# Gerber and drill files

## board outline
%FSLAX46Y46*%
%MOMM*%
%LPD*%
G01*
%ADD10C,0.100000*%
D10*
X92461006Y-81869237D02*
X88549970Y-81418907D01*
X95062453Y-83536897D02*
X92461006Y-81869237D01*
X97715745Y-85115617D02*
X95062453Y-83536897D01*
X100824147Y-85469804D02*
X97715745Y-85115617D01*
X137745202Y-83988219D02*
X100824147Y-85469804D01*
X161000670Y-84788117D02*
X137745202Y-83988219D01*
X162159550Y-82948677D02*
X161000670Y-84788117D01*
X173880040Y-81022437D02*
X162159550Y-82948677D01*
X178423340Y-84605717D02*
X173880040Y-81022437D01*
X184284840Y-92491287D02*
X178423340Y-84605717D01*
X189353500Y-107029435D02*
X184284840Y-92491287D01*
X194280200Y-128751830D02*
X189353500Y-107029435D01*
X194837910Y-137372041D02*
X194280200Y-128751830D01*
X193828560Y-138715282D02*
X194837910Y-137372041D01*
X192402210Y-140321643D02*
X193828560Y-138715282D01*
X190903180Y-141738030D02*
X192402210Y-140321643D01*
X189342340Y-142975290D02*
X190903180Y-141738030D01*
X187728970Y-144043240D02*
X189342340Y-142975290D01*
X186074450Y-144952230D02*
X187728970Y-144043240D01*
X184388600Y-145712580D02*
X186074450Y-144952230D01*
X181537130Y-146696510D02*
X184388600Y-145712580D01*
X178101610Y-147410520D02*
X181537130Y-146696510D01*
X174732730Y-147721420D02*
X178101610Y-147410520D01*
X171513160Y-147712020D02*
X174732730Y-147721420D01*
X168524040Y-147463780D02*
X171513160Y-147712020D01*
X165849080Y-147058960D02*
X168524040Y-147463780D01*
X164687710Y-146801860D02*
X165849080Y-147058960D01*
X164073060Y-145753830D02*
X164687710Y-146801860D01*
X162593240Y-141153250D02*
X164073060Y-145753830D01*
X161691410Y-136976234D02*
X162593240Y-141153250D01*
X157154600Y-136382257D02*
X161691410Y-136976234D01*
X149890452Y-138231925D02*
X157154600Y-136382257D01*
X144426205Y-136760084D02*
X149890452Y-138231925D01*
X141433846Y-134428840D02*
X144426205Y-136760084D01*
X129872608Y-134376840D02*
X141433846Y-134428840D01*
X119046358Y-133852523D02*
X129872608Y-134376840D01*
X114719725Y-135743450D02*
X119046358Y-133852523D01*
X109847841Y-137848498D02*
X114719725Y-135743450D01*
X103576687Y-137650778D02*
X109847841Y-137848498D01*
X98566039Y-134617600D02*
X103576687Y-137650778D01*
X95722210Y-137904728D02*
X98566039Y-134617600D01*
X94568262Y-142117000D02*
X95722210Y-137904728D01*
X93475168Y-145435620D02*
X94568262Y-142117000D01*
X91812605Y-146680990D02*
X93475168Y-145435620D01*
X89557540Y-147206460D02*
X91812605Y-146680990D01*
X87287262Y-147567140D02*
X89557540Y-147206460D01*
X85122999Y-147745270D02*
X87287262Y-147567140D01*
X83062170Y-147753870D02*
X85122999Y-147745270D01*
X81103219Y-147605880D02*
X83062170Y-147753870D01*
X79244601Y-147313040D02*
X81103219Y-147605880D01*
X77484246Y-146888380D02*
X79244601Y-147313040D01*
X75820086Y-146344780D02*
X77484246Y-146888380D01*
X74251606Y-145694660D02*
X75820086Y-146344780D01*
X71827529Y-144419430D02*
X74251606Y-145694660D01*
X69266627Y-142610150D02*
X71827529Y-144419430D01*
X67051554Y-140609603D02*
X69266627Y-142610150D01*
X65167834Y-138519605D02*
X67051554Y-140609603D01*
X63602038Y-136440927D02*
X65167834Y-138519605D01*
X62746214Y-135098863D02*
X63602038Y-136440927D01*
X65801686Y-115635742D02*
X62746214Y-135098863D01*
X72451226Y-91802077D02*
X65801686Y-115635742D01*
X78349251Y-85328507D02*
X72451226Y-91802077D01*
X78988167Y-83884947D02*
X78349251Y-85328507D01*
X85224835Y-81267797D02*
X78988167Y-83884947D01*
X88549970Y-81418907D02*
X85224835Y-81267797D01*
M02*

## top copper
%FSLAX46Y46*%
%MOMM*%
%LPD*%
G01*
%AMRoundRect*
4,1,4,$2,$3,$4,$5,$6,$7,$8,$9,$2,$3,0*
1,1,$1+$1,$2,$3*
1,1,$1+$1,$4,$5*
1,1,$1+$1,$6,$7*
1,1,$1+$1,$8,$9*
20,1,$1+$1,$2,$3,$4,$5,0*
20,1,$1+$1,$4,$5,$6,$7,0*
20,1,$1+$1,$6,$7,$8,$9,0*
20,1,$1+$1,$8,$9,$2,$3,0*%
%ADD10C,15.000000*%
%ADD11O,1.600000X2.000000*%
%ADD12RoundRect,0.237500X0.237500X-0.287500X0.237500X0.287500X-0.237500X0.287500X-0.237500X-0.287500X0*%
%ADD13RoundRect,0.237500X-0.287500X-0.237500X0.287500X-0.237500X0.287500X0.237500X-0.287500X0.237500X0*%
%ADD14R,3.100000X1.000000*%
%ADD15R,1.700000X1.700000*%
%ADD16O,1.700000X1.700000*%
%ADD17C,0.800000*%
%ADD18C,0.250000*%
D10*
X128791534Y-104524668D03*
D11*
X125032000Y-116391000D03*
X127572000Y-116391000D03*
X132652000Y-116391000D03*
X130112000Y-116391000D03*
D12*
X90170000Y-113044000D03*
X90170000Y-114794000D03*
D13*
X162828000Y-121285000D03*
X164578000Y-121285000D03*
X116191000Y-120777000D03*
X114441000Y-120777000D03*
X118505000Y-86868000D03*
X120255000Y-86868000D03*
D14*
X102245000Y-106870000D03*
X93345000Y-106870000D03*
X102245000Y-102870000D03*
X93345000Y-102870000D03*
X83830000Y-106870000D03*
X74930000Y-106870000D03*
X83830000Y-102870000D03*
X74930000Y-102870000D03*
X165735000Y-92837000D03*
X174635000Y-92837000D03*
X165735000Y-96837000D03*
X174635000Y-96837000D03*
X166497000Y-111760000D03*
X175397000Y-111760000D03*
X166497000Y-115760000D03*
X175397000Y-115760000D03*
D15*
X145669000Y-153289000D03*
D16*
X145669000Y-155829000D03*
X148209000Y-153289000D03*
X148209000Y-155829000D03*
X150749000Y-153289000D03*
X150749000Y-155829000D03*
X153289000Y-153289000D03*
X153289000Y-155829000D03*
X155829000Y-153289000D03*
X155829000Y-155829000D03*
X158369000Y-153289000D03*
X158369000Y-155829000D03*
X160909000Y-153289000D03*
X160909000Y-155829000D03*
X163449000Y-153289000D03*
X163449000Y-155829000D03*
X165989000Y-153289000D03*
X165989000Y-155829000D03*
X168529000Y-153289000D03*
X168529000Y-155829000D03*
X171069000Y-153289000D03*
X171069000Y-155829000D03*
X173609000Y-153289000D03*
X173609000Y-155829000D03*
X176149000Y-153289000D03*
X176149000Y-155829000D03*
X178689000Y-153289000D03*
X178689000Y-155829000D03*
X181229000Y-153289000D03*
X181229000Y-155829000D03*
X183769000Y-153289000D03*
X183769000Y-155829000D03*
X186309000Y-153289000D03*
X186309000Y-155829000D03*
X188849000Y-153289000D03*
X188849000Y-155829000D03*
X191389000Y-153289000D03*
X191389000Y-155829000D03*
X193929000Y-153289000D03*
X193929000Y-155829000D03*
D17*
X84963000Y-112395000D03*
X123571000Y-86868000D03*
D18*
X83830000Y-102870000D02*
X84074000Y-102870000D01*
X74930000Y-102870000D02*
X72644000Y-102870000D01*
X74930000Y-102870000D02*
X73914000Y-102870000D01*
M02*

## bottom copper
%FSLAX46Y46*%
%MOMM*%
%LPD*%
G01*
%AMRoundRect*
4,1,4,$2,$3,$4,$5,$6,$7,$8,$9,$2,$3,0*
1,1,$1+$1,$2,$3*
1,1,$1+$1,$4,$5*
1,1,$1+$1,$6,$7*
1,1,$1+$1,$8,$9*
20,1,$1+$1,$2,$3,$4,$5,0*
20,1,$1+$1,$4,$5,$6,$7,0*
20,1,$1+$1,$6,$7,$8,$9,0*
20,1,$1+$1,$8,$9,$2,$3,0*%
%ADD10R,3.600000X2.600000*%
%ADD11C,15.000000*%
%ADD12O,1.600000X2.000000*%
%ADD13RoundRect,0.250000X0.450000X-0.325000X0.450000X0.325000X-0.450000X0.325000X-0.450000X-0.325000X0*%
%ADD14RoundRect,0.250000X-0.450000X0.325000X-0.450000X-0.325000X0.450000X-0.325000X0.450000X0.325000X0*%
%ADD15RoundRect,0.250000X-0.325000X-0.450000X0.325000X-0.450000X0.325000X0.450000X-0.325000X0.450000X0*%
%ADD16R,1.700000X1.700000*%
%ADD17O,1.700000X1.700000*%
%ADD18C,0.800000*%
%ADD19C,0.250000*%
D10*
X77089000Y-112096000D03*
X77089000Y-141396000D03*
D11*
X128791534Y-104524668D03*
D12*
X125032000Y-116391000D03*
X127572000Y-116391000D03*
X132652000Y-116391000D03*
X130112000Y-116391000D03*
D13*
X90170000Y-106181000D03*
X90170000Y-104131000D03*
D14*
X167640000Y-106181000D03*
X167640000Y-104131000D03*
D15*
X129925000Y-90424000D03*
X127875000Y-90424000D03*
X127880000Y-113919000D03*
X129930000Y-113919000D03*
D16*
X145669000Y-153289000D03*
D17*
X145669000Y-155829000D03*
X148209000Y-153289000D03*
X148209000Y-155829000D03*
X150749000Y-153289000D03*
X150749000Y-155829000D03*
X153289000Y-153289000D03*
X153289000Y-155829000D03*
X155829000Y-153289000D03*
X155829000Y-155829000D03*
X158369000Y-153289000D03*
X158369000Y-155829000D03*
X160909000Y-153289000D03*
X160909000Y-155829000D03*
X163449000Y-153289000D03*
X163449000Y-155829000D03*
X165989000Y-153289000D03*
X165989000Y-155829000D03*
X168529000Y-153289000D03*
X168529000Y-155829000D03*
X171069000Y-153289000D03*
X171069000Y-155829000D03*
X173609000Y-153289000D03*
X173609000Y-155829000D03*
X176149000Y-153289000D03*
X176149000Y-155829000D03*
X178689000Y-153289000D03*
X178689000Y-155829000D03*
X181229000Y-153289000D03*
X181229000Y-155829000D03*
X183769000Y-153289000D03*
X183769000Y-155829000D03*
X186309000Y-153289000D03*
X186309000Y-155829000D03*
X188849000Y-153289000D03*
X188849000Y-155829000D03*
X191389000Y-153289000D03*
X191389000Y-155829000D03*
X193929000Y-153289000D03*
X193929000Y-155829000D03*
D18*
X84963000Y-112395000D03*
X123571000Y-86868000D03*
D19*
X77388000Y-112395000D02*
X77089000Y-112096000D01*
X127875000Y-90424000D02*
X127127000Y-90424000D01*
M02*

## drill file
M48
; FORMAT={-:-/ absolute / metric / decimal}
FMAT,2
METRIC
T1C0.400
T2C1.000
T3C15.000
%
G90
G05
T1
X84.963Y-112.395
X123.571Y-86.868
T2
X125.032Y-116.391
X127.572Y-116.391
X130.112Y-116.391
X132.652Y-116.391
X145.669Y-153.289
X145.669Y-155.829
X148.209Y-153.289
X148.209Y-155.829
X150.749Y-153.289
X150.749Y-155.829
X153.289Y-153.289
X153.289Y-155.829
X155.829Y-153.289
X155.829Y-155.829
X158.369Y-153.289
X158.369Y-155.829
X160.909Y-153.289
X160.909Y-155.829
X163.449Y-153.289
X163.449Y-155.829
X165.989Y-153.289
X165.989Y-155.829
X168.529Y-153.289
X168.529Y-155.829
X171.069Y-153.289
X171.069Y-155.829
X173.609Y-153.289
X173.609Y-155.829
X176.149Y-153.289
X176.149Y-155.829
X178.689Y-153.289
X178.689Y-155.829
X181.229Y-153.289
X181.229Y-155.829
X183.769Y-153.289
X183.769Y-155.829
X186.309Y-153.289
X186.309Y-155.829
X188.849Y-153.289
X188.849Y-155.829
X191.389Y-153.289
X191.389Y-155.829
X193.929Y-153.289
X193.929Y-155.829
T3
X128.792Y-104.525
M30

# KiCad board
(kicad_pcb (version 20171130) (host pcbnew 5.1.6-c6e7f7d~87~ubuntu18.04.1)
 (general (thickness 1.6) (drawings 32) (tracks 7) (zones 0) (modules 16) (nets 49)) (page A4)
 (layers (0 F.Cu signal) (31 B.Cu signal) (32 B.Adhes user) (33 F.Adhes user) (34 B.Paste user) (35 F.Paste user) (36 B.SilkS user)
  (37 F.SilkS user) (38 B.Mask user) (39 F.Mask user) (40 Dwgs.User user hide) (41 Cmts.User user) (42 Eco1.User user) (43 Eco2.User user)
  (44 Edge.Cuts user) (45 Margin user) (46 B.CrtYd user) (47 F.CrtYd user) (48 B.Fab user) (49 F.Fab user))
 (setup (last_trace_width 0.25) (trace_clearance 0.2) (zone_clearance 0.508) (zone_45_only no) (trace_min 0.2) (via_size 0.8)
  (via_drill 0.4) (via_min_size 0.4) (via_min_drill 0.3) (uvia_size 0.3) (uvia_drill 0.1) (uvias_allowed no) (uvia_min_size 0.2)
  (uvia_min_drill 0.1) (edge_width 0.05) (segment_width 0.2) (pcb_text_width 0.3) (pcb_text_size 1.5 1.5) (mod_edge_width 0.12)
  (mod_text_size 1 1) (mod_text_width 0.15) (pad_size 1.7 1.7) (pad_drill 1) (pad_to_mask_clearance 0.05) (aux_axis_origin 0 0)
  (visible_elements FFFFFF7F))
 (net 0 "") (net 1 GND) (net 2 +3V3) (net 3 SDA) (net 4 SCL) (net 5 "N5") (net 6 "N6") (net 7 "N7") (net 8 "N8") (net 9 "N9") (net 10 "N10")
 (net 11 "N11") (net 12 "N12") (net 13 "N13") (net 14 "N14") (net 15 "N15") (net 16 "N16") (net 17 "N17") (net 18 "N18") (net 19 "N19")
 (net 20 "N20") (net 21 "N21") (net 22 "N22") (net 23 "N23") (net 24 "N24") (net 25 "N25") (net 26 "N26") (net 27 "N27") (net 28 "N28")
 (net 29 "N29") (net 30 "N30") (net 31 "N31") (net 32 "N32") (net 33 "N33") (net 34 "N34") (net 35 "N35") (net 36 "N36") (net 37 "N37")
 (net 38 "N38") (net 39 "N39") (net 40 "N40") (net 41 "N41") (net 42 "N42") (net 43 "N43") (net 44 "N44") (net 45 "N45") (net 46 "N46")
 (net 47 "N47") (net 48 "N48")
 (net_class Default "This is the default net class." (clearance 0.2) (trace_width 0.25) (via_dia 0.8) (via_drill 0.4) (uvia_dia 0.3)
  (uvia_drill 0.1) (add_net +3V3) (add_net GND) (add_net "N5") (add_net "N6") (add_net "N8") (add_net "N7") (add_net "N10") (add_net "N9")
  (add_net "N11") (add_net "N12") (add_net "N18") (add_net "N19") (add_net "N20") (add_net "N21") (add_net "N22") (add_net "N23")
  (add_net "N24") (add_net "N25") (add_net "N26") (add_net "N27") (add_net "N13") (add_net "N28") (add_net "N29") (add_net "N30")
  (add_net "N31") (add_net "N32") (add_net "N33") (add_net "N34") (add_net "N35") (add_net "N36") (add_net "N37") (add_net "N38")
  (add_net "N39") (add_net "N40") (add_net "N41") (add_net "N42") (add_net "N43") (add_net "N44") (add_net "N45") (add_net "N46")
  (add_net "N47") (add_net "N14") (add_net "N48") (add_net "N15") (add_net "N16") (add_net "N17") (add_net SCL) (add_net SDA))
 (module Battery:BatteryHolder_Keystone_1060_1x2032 (layer B.Cu) (at 77.089 126.746 90)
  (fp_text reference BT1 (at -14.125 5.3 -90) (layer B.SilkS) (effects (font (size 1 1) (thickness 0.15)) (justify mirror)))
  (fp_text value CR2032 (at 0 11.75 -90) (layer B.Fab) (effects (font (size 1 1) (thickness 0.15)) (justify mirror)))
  (pad 2 smd rect (at 14.65 0 270) (size 2.6 3.6) (layers B.Cu B.Paste B.Mask) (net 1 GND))
  (pad 1 smd rect (at -14.65 0 270) (size 2.6 3.6) (layers B.Cu B.Paste B.Mask) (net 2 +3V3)))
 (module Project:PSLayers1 (layer F.Cu) (at 127 115.824)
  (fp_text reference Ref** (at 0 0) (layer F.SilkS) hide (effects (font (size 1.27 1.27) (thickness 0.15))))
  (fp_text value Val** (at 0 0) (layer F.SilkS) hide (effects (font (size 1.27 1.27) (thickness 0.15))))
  (fp_line (start -34.538994 -33.954763) (end -38.45003 -34.405093) (layer Edge.Cuts) (width 0.1))
  (fp_line (start -31.937547 -32.287103) (end -34.538994 -33.954763) (layer Edge.Cuts) (width 0.1))
  (fp_line (start -29.284255 -30.708383) (end -31.937547 -32.287103) (layer Edge.Cuts) (width 0.1))
  (fp_line (start -26.175853 -30.354196) (end -29.284255 -30.708383) (layer Edge.Cuts) (width 0.1))
  (fp_line (start 10.745202 -31.835781) (end -26.175853 -30.354196) (layer Edge.Cuts) (width 0.1))
  (fp_line (start 34.00067 -31.035883) (end 10.745202 -31.835781) (layer Edge.Cuts) (width 0.1))
  (fp_line (start 35.15955 -32.875323) (end 34.00067 -31.035883) (layer Edge.Cuts) (width 0.1))
  (fp_line (start 46.88004 -34.801563) (end 35.15955 -32.875323) (layer Edge.Cuts) (width 0.1))
  (fp_line (start 51.42334 -31.218283) (end 46.88004 -34.801563) (layer Edge.Cuts) (width 0.1))
  (fp_line (start 57.28484 -23.332713) (end 51.42334 -31.218283) (layer Edge.Cuts) (width 0.1))
  (fp_line (start 62.3535 -8.794565) (end 57.28484 -23.332713) (layer Edge.Cuts) (width 0.1))
  (fp_line (start 67.2802 12.92783) (end 62.3535 -8.794565) (layer Edge.Cuts) (width 0.1))
  (fp_line (start 67.83791 21.548041) (end 67.2802 12.92783) (layer Edge.Cuts) (width 0.1))
  (fp_line (start 66.82856 22.891282) (end 67.83791 21.548041) (layer Edge.Cuts) (width 0.1))
  (fp_line (start 65.40221 24.497643) (end 66.82856 22.891282) (layer Edge.Cuts) (width 0.1))
  (fp_line (start 63.90318 25.91403) (end 65.40221 24.497643) (layer Edge.Cuts) (width 0.1))
  (fp_line (start 62.34234 27.15129) (end 63.90318 25.91403) (layer Edge.Cuts) (width 0.1))
  (fp_line (start 60.72897 28.21924) (end 62.34234 27.15129) (layer Edge.Cuts) (width 0.1))
  (fp_line (start 59.07445 29.12823) (end 60.72897 28.21924) (layer Edge.Cuts) (width 0.1))
  (fp_line (start 57.3886 29.88858) (end 59.07445 29.12823) (layer Edge.Cuts) (width 0.1))
  (fp_line (start 54.53713 30.87251) (end 57.3886 29.88858) (layer Edge.Cuts) (width 0.1))
  (fp_line (start 51.10161 31.58652) (end 54.53713 30.87251) (layer Edge.Cuts) (width 0.1))
  (fp_line (start 47.73273 31.89742) (end 51.10161 31.58652) (layer Edge.Cuts) (width 0.1))
  (fp_line (start 44.51316 31.88802) (end 47.73273 31.89742) (layer Edge.Cuts) (width 0.1))
  (fp_line (start 41.52404 31.63978) (end 44.51316 31.88802) (layer Edge.Cuts) (width 0.1))
  (fp_line (start 38.84908 31.23496) (end 41.52404 31.63978) (layer Edge.Cuts) (width 0.1))
  (fp_line (start 37.68771 30.97786) (end 38.84908 31.23496) (layer Edge.Cuts) (width 0.1))
  (fp_line (start 37.07306 29.92983) (end 37.68771 30.97786) (layer Edge.Cuts) (width 0.1))
  (fp_line (start 35.59324 25.32925) (end 37.07306 29.92983) (layer Edge.Cuts) (width 0.1))
  (fp_line (start 34.69141 21.152234) (end 35.59324 25.32925) (layer Edge.Cuts) (width 0.1))
  (fp_line (start 30.1546 20.558257) (end 34.69141 21.152234) (layer Edge.Cuts) (width 0.1))
  (fp_line (start 22.890452 22.407925) (end 30.1546 20.558257) (layer Edge.Cuts) (width 0.1))
  (fp_line (start 17.426205 20.936084) (end 22.890452 22.407925) (layer Edge.Cuts) (width 0.1))
  (fp_line (start 14.433846 18.60484) (end 17.426205 20.936084) (layer Edge.Cuts) (width 0.1))
  (fp_line (start 2.872608 18.55284) (end 14.433846 18.60484) (layer Edge.Cuts) (width 0.1))
  (fp_line (start -7.953642 18.028523) (end 2.872608 18.55284) (layer Edge.Cuts) (width 0.1))
  (fp_line (start -12.280275 19.91945) (end -7.953642 18.028523) (layer Edge.Cuts) (width 0.1))
  (fp_line (start -17.152159 22.024498) (end -12.280275 19.91945) (layer Edge.Cuts) (width 0.1))
  (fp_line (start -23.423313 21.826778) (end -17.152159 22.024498) (layer Edge.Cuts) (width 0.1))
  (fp_line (start -28.433961 18.7936) (end -23.423313 21.826778) (layer Edge.Cuts) (width 0.1))
  (fp_line (start -31.27779 22.080728) (end -28.433961 18.7936) (layer Edge.Cuts) (width 0.1))
  (fp_line (start -32.431738 26.293) (end -31.27779 22.080728) (layer Edge.Cuts) (width 0.1))
  (fp_line (start -33.524832 29.61162) (end -32.431738 26.293) (layer Edge.Cuts) (width 0.1))
  (fp_line (start -35.187395 30.85699) (end -33.524832 29.61162) (layer Edge.Cuts) (width 0.1))
  (fp_line (start -37.44246 31.38246) (end -35.187395 30.85699) (layer Edge.Cuts) (width 0.1))
  (fp_line (start -39.712738 31.74314) (end -37.44246 31.38246) (layer Edge.Cuts) (width 0.1))
  (fp_line (start -41.877001 31.92127) (end -39.712738 31.74314) (layer Edge.Cuts) (width 0.1))
  (fp_line (start -43.93783 31.92987) (end -41.877001 31.92127) (layer Edge.Cuts) (width 0.1))
  (fp_line (start -45.896781 31.78188) (end -43.93783 31.92987) (layer Edge.Cuts) (width 0.1))
  (fp_line (start -47.755399 31.48904) (end -45.896781 31.78188) (layer Edge.Cuts) (width 0.1))
  (fp_line (start -49.515754 31.06438) (end -47.755399 31.48904) (layer Edge.Cuts) (width 0.1))
  (fp_line (start -51.179914 30.52078) (end -49.515754 31.06438) (layer Edge.Cuts) (width 0.1))
  (fp_line (start -52.748394 29.87066) (end -51.179914 30.52078) (layer Edge.Cuts) (width 0.1))
  (fp_line (start -55.172471 28.59543) (end -52.748394 29.87066) (layer Edge.Cuts) (width 0.1))
  (fp_line (start -57.733373 26.78615) (end -55.172471 28.59543) (layer Edge.Cuts) (width 0.1))
  (fp_line (start -59.948446 24.785603) (end -57.733373 26.78615) (layer Edge.Cuts) (width 0.1))
  (fp_line (start -61.832166 22.695605) (end -59.948446 24.785603) (layer Edge.Cuts) (width 0.1))
  (fp_line (start -63.397962 20.616927) (end -61.832166 22.695605) (layer Edge.Cuts) (width 0.1))
  (fp_line (start -64.253786 19.274863) (end -63.397962 20.616927) (layer Edge.Cuts) (width 0.1))
  (fp_line (start -61.198314 -0.188258) (end -64.253786 19.274863) (layer Edge.Cuts) (width 0.1))
  (fp_line (start -54.548774 -24.021923) (end -61.198314 -0.188258) (layer Edge.Cuts) (width 0.1))
  (fp_line (start -48.650749 -30.495493) (end -54.548774 -24.021923) (layer Edge.Cuts) (width 0.1))
  (fp_line (start -48.011833 -31.939053) (end -48.650749 -30.495493) (layer Edge.Cuts) (width 0.1))
  (fp_line (start -41.775165 -34.556203) (end -48.011833 -31.939053) (layer Edge.Cuts) (width 0.1))
  (fp_line (start -38.45003 -34.405093) (end -41.775165 -34.556203) (layer Edge.Cuts) (width 0.1))
  (pad 1 thru_hole circle (at 1.791534 -11.299332) (size 15 15) (drill 15) (layers *.Cu *.Mask)))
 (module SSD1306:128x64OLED (layer F.Cu) (at 129.032 105.791 180)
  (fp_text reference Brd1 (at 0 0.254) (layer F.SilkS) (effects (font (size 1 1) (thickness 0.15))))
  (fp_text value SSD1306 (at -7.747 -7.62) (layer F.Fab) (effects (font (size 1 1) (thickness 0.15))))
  (pad 4 thru_hole oval (at 4 -10.6 270) (size 2 1.6) (drill 1) (layers *.Cu *.Mask) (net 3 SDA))
  (pad 3 thru_hole oval (at 1.46 -10.6 270) (size 2 1.6) (drill 1) (layers *.Cu *.Mask) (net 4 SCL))
  (pad 1 thru_hole oval (at -3.62 -10.6 270) (size 2 1.6) (drill 1) (layers *.Cu *.Mask) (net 1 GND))
  (pad 2 thru_hole oval (at -1.08 -10.6 270) (size 2 1.6) (drill 1) (layers *.Cu *.Mask) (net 2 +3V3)))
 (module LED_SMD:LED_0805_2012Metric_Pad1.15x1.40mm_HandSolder (layer B.Cu) (at 90.17 105.156 90)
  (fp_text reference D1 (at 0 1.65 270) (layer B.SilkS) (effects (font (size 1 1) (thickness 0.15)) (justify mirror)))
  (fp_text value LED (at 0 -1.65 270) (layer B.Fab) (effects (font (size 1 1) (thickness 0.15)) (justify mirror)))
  (pad 1 smd roundrect (at -1.025 0 90) (size 1.15 1.4) (layers B.Cu B.Paste B.Mask) (roundrect_rratio 0.217391) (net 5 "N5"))
  (pad 2 smd roundrect (at 1.025 0 90) (size 1.15 1.4) (layers B.Cu B.Paste B.Mask) (roundrect_rratio 0.217391) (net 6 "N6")))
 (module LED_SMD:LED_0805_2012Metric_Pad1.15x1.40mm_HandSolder (layer B.Cu) (at 167.64 105.156 270)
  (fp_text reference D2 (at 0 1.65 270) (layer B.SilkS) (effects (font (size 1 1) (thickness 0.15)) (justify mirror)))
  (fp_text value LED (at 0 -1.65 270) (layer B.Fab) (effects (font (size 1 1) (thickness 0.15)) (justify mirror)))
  (pad 2 smd roundrect (at 1.025 0 270) (size 1.15 1.4) (layers B.Cu B.Paste B.Mask) (roundrect_rratio 0.217391) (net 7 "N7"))
  (pad 1 smd roundrect (at -1.025 0 270) (size 1.15 1.4) (layers B.Cu B.Paste B.Mask) (roundrect_rratio 0.217391) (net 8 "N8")))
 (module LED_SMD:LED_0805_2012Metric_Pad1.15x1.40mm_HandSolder (layer B.Cu) (at 128.9 90.424)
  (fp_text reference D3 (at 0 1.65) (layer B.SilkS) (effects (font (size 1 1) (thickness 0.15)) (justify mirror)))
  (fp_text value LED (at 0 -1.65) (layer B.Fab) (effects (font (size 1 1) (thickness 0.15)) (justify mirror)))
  (pad 2 smd roundrect (at 1.025 0) (size 1.15 1.4) (layers B.Cu B.Paste B.Mask) (roundrect_rratio 0.217391) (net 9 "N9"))
  (pad 1 smd roundrect (at -1.025 0) (size 1.15 1.4) (layers B.Cu B.Paste B.Mask) (roundrect_rratio 0.217391) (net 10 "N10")))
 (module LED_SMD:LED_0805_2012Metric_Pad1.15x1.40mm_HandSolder (layer B.Cu) (at 128.905 113.919)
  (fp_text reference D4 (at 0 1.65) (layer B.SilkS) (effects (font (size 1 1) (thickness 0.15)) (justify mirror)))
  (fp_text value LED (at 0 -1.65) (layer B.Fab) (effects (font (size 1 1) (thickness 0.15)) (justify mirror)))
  (pad 1 smd roundrect (at -1.025 0) (size 1.15 1.4) (layers B.Cu B.Paste B.Mask) (roundrect_rratio 0.217391) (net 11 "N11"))
  (pad 2 smd roundrect (at 1.025 0) (size 1.15 1.4) (layers B.Cu B.Paste B.Mask) (roundrect_rratio 0.217391) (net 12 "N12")))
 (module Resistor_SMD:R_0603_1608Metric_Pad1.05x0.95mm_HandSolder (layer F.Cu) (at 90.17 113.919 90)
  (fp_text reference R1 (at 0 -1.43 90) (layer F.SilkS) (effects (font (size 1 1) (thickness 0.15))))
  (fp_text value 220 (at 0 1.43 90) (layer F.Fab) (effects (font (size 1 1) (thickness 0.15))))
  (pad 2 smd roundrect (at 0.875 0 90) (size 1.05 0.95) (layers F.Cu F.Paste F.Mask) (roundrect_rratio 0.25) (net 5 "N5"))
  (pad 1 smd roundrect (at -0.875 0 90) (size 1.05 0.95) (layers F.Cu F.Paste F.Mask) (roundrect_rratio 0.25) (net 1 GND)))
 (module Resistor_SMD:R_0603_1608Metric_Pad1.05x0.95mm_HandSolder (layer F.Cu) (at 163.703 121.285)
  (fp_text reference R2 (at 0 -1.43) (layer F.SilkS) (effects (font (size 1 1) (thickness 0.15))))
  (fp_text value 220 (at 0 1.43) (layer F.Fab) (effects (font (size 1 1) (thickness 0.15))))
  (pad 1 smd roundrect (at -0.875 0) (size 1.05 0.95) (layers F.Cu F.Paste F.Mask) (roundrect_rratio 0.25) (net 1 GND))
  (pad 2 smd roundrect (at 0.875 0) (size 1.05 0.95) (layers F.Cu F.Paste F.Mask) (roundrect_rratio 0.25) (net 8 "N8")))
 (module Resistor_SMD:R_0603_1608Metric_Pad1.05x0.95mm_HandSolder (layer F.Cu) (at 115.316 120.777)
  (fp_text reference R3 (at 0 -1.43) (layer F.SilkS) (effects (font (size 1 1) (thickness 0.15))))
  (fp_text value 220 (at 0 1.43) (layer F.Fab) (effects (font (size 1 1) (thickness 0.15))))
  (pad 2 smd roundrect (at 0.875 0) (size 1.05 0.95) (layers F.Cu F.Paste F.Mask) (roundrect_rratio 0.25) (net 11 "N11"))
  (pad 1 smd roundrect (at -0.875 0) (size 1.05 0.95) (layers F.Cu F.Paste F.Mask) (roundrect_rratio 0.25) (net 1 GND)))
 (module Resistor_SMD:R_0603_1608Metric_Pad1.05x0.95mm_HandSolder (layer F.Cu) (at 119.38 86.868)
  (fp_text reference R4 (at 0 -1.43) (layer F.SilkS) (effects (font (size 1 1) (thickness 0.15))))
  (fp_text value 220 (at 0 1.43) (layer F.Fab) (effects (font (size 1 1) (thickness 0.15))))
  (pad 1 smd roundrect (at -0.875 0) (size 1.05 0.95) (layers F.Cu F.Paste F.Mask) (roundrect_rratio 0.25) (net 1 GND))
  (pad 2 smd roundrect (at 0.875 0) (size 1.05 0.95) (layers F.Cu F.Paste F.Mask) (roundrect_rratio 0.25) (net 10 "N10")))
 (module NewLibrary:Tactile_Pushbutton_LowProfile (layer F.Cu) (at 98.425 111.76)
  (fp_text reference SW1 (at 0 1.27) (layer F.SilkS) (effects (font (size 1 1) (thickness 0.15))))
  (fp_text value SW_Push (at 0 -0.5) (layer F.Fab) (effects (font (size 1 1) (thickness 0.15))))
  (pad 4 smd rect (at 3.82 -4.89) (size 3.1 1) (layers F.Cu F.Paste F.Mask))
  (pad 3 smd rect (at -5.08 -4.89) (size 3.1 1) (layers F.Cu F.Paste F.Mask))
  (pad 2 smd rect (at 3.82 -8.89 90) (size 1 3.1) (layers F.Cu F.Paste F.Mask) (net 7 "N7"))
  (pad 1 smd rect (at -5.08 -8.89 90) (size 1 3.1) (layers F.Cu F.Paste F.Mask) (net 2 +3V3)))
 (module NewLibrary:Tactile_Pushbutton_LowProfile (layer F.Cu) (at 80.01 111.76)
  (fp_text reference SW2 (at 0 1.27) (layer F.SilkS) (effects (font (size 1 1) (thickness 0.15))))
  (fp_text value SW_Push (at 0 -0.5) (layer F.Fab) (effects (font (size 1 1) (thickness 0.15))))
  (pad 4 smd rect (at 3.82 -4.89) (size 3.1 1) (layers F.Cu F.Paste F.Mask))
  (pad 3 smd rect (at -5.08 -4.89) (size 3.1 1) (layers F.Cu F.Paste F.Mask))
  (pad 2 smd rect (at 3.82 -8.89 90) (size 1 3.1) (layers F.Cu F.Paste F.Mask) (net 6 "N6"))
  (pad 1 smd rect (at -5.08 -8.89 90) (size 1 3.1) (layers F.Cu F.Paste F.Mask) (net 2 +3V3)))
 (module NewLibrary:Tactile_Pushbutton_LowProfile (layer F.Cu) (at 170.815 101.727)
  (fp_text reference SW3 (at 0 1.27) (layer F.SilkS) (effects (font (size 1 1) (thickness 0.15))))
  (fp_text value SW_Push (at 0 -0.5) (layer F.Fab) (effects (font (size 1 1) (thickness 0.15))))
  (pad 1 smd rect (at -5.08 -8.89 90) (size 1 3.1) (layers F.Cu F.Paste F.Mask) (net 9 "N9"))
  (pad 2 smd rect (at 3.82 -8.89 90) (size 1 3.1) (layers F.Cu F.Paste F.Mask) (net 2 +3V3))
  (pad 3 smd rect (at -5.08 -4.89) (size 3.1 1) (layers F.Cu F.Paste F.Mask))
  (pad 4 smd rect (at 3.82 -4.89) (size 3.1 1) (layers F.Cu F.Paste F.Mask)))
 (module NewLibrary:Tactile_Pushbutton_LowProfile (layer F.Cu) (at 171.577 120.65)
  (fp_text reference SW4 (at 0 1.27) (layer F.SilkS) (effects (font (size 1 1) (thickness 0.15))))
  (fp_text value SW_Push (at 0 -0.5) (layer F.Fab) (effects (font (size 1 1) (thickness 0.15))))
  (pad 1 smd rect (at -5.08 -8.89 90) (size 1 3.1) (layers F.Cu F.Paste F.Mask) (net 2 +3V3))
  (pad 2 smd rect (at 3.82 -8.89 90) (size 1 3.1) (layers F.Cu F.Paste F.Mask) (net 12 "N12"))
  (pad 3 smd rect (at -5.08 -4.89) (size 3.1 1) (layers F.Cu F.Paste F.Mask))
  (pad 4 smd rect (at 3.82 -4.89) (size 3.1 1) (layers F.Cu F.Paste F.Mask)))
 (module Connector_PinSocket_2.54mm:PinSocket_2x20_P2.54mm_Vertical (layer F.Cu) (at 145.669 153.289 90)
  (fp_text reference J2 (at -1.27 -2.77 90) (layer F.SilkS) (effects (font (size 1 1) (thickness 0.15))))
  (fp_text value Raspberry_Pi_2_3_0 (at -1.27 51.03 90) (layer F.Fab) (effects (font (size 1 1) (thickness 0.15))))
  (pad 1 thru_hole rect (at 0 0 90) (size 1.7 1.7) (drill 1) (layers *.Cu *.Mask) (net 2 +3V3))
  (pad 2 thru_hole oval (at -2.54 0 90) (size 1.7 1.7) (drill 1) (layers *.Cu *.Mask) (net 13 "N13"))
  (pad 3 thru_hole oval (at 0 2.54 90) (size 1.7 1.7) (drill 1) (layers *.Cu *.Mask) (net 3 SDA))
  (pad 4 thru_hole oval (at -2.54 2.54 90) (size 1.7 1.7) (drill 1) (layers *.Cu *.Mask) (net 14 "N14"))
  (pad 5 thru_hole oval (at 0 5.08 90) (size 1.7 1.7) (drill 1) (layers *.Cu *.Mask) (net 4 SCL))
  (pad 6 thru_hole oval (at -2.54 5.08 90) (size 1.7 1.7) (drill 1) (layers *.Cu *.Mask) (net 1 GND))
  (pad 7 thru_hole oval (at 0 7.62 90) (size 1.7 1.7) (drill 1) (layers *.Cu *.Mask) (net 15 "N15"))
  (pad 8 thru_hole oval (at -2.54 7.62 90) (size 1.7 1.7) (drill 1) (layers *.Cu *.Mask) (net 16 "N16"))
  (pad 9 thru_hole oval (at 0 10.16 90) (size 1.7 1.7) (drill 1) (layers *.Cu *.Mask) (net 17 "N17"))
  (pad 10 thru_hole oval (at -2.54 10.16 90) (size 1.7 1.7) (drill 1) (layers *.Cu *.Mask) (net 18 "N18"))
  (pad 11 thru_hole oval (at 0 12.7 90) (size 1.7 1.7) (drill 1) (layers *.Cu *.Mask) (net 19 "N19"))
  (pad 12 thru_hole oval (at -2.54 12.7 90) (size 1.7 1.7) (drill 1) (layers *.Cu *.Mask) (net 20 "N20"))
  (pad 13 thru_hole oval (at 0 15.24 90) (size 1.7 1.7) (drill 1) (layers *.Cu *.Mask) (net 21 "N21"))
  (pad 14 thru_hole oval (at -2.54 15.24 90) (size 1.7 1.7) (drill 1) (layers *.Cu *.Mask) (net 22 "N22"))
  (pad 15 thru_hole oval (at 0 17.78 90) (size 1.7 1.7) (drill 1) (layers *.Cu *.Mask) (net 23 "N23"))
  (pad 16 thru_hole oval (at -2.54 17.78 90) (size 1.7 1.7) (drill 1) (layers *.Cu *.Mask) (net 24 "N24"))
  (pad 17 thru_hole oval (at 0 20.32 90) (size 1.7 1.7) (drill 1) (layers *.Cu *.Mask) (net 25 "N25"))
  (pad 18 thru_hole oval (at -2.54 20.32 90) (size 1.7 1.7) (drill 1) (layers *.Cu *.Mask) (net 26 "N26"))
  (pad 19 thru_hole oval (at 0 22.86 90) (size 1.7 1.7) (drill 1) (layers *.Cu *.Mask) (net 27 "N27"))
  (pad 20 thru_hole oval (at -2.54 22.86 90) (size 1.7 1.7) (drill 1) (layers *.Cu *.Mask) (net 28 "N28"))
  (pad 21 thru_hole oval (at 0 25.4 90) (size 1.7 1.7) (drill 1) (layers *.Cu *.Mask) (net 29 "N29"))
  (pad 22 thru_hole oval (at -2.54 25.4 90) (size 1.7 1.7) (drill 1) (layers *.Cu *.Mask) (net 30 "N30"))
  (pad 23 thru_hole oval (at 0 27.94 90) (size 1.7 1.7) (drill 1) (layers *.Cu *.Mask) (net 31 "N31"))
  (pad 24 thru_hole oval (at -2.54 27.94 90) (size 1.7 1.7) (drill 1) (layers *.Cu *.Mask) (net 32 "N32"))
  (pad 25 thru_hole oval (at 0 30.48 90) (size 1.7 1.7) (drill 1) (layers *.Cu *.Mask) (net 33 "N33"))
  (pad 26 thru_hole oval (at -2.54 30.48 90) (size 1.7 1.7) (drill 1) (layers *.Cu *.Mask) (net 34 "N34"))
  (pad 27 thru_hole oval (at 0 33.02 90) (size 1.7 1.7) (drill 1) (layers *.Cu *.Mask) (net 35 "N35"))
  (pad 28 thru_hole oval (at -2.54 33.02 90) (size 1.7 1.7) (drill 1) (layers *.Cu *.Mask) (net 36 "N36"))
  (pad 29 thru_hole oval (at 0 35.56 90) (size 1.7 1.7) (drill 1) (layers *.Cu *.Mask) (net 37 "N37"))
  (pad 30 thru_hole oval (at -2.54 35.56 90) (size 1.7 1.7) (drill 1) (layers *.Cu *.Mask) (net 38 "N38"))
  (pad 31 thru_hole oval (at 0 38.1 90) (size 1.7 1.7) (drill 1) (layers *.Cu *.Mask) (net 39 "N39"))
  (pad 32 thru_hole oval (at -2.54 38.1 90) (size 1.7 1.7) (drill 1) (layers *.Cu *.Mask) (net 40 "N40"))
  (pad 33 thru_hole oval (at 0 40.64 90) (size 1.7 1.7) (drill 1) (layers *.Cu *.Mask) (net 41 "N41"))
  (pad 34 thru_hole oval (at -2.54 40.64 90) (size 1.7 1.7) (drill 1) (layers *.Cu *.Mask) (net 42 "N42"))
  (pad 35 thru_hole oval (at 0 43.18 90) (size 1.7 1.7) (drill 1) (layers *.Cu *.Mask) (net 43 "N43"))
  (pad 36 thru_hole oval (at -2.54 43.18 90) (size 1.7 1.7) (drill 1) (layers *.Cu *.Mask) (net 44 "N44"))
  (pad 37 thru_hole oval (at 0 45.72 90) (size 1.7 1.7) (drill 1) (layers *.Cu *.Mask) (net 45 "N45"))
  (pad 38 thru_hole oval (at -2.54 45.72 90) (size 1.7 1.7) (drill 1) (layers *.Cu *.Mask) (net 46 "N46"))
  (pad 39 thru_hole oval (at 0 48.26 90) (size 1.7 1.7) (drill 1) (layers *.Cu *.Mask) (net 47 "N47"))
  (pad 40 thru_hole oval (at -2.54 48.26 90) (size 1.7 1.7) (drill 1) (layers *.Cu *.Mask) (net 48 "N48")))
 (via (at 84.963 112.395) (size 0.8) (drill 0.4) (layers F.Cu B.Cu) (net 1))
 (segment (start 77.388 112.395) (end 77.089 112.096) (width 0.25) (layer B.Cu) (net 1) (status 30))
 (segment (start 83.83 102.87) (end 84.074 102.87) (width 0.25) (layer F.Cu) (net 6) (status 30))
 (via (at 123.571 86.868) (size 0.8) (drill 0.4) (layers F.Cu B.Cu) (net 10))
 (segment (start 127.875 90.424) (end 127.127 90.424) (width 0.25) (layer B.Cu) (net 10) (status 10))
 (segment (start 74.93 102.87) (end 72.644 102.87) (width 0.25) (layer F.Cu) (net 2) (status 10))
 (segment (start 74.93 102.87) (end 73.914 102.87) (width 0.25) (layer F.Cu) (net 2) (status 30)))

